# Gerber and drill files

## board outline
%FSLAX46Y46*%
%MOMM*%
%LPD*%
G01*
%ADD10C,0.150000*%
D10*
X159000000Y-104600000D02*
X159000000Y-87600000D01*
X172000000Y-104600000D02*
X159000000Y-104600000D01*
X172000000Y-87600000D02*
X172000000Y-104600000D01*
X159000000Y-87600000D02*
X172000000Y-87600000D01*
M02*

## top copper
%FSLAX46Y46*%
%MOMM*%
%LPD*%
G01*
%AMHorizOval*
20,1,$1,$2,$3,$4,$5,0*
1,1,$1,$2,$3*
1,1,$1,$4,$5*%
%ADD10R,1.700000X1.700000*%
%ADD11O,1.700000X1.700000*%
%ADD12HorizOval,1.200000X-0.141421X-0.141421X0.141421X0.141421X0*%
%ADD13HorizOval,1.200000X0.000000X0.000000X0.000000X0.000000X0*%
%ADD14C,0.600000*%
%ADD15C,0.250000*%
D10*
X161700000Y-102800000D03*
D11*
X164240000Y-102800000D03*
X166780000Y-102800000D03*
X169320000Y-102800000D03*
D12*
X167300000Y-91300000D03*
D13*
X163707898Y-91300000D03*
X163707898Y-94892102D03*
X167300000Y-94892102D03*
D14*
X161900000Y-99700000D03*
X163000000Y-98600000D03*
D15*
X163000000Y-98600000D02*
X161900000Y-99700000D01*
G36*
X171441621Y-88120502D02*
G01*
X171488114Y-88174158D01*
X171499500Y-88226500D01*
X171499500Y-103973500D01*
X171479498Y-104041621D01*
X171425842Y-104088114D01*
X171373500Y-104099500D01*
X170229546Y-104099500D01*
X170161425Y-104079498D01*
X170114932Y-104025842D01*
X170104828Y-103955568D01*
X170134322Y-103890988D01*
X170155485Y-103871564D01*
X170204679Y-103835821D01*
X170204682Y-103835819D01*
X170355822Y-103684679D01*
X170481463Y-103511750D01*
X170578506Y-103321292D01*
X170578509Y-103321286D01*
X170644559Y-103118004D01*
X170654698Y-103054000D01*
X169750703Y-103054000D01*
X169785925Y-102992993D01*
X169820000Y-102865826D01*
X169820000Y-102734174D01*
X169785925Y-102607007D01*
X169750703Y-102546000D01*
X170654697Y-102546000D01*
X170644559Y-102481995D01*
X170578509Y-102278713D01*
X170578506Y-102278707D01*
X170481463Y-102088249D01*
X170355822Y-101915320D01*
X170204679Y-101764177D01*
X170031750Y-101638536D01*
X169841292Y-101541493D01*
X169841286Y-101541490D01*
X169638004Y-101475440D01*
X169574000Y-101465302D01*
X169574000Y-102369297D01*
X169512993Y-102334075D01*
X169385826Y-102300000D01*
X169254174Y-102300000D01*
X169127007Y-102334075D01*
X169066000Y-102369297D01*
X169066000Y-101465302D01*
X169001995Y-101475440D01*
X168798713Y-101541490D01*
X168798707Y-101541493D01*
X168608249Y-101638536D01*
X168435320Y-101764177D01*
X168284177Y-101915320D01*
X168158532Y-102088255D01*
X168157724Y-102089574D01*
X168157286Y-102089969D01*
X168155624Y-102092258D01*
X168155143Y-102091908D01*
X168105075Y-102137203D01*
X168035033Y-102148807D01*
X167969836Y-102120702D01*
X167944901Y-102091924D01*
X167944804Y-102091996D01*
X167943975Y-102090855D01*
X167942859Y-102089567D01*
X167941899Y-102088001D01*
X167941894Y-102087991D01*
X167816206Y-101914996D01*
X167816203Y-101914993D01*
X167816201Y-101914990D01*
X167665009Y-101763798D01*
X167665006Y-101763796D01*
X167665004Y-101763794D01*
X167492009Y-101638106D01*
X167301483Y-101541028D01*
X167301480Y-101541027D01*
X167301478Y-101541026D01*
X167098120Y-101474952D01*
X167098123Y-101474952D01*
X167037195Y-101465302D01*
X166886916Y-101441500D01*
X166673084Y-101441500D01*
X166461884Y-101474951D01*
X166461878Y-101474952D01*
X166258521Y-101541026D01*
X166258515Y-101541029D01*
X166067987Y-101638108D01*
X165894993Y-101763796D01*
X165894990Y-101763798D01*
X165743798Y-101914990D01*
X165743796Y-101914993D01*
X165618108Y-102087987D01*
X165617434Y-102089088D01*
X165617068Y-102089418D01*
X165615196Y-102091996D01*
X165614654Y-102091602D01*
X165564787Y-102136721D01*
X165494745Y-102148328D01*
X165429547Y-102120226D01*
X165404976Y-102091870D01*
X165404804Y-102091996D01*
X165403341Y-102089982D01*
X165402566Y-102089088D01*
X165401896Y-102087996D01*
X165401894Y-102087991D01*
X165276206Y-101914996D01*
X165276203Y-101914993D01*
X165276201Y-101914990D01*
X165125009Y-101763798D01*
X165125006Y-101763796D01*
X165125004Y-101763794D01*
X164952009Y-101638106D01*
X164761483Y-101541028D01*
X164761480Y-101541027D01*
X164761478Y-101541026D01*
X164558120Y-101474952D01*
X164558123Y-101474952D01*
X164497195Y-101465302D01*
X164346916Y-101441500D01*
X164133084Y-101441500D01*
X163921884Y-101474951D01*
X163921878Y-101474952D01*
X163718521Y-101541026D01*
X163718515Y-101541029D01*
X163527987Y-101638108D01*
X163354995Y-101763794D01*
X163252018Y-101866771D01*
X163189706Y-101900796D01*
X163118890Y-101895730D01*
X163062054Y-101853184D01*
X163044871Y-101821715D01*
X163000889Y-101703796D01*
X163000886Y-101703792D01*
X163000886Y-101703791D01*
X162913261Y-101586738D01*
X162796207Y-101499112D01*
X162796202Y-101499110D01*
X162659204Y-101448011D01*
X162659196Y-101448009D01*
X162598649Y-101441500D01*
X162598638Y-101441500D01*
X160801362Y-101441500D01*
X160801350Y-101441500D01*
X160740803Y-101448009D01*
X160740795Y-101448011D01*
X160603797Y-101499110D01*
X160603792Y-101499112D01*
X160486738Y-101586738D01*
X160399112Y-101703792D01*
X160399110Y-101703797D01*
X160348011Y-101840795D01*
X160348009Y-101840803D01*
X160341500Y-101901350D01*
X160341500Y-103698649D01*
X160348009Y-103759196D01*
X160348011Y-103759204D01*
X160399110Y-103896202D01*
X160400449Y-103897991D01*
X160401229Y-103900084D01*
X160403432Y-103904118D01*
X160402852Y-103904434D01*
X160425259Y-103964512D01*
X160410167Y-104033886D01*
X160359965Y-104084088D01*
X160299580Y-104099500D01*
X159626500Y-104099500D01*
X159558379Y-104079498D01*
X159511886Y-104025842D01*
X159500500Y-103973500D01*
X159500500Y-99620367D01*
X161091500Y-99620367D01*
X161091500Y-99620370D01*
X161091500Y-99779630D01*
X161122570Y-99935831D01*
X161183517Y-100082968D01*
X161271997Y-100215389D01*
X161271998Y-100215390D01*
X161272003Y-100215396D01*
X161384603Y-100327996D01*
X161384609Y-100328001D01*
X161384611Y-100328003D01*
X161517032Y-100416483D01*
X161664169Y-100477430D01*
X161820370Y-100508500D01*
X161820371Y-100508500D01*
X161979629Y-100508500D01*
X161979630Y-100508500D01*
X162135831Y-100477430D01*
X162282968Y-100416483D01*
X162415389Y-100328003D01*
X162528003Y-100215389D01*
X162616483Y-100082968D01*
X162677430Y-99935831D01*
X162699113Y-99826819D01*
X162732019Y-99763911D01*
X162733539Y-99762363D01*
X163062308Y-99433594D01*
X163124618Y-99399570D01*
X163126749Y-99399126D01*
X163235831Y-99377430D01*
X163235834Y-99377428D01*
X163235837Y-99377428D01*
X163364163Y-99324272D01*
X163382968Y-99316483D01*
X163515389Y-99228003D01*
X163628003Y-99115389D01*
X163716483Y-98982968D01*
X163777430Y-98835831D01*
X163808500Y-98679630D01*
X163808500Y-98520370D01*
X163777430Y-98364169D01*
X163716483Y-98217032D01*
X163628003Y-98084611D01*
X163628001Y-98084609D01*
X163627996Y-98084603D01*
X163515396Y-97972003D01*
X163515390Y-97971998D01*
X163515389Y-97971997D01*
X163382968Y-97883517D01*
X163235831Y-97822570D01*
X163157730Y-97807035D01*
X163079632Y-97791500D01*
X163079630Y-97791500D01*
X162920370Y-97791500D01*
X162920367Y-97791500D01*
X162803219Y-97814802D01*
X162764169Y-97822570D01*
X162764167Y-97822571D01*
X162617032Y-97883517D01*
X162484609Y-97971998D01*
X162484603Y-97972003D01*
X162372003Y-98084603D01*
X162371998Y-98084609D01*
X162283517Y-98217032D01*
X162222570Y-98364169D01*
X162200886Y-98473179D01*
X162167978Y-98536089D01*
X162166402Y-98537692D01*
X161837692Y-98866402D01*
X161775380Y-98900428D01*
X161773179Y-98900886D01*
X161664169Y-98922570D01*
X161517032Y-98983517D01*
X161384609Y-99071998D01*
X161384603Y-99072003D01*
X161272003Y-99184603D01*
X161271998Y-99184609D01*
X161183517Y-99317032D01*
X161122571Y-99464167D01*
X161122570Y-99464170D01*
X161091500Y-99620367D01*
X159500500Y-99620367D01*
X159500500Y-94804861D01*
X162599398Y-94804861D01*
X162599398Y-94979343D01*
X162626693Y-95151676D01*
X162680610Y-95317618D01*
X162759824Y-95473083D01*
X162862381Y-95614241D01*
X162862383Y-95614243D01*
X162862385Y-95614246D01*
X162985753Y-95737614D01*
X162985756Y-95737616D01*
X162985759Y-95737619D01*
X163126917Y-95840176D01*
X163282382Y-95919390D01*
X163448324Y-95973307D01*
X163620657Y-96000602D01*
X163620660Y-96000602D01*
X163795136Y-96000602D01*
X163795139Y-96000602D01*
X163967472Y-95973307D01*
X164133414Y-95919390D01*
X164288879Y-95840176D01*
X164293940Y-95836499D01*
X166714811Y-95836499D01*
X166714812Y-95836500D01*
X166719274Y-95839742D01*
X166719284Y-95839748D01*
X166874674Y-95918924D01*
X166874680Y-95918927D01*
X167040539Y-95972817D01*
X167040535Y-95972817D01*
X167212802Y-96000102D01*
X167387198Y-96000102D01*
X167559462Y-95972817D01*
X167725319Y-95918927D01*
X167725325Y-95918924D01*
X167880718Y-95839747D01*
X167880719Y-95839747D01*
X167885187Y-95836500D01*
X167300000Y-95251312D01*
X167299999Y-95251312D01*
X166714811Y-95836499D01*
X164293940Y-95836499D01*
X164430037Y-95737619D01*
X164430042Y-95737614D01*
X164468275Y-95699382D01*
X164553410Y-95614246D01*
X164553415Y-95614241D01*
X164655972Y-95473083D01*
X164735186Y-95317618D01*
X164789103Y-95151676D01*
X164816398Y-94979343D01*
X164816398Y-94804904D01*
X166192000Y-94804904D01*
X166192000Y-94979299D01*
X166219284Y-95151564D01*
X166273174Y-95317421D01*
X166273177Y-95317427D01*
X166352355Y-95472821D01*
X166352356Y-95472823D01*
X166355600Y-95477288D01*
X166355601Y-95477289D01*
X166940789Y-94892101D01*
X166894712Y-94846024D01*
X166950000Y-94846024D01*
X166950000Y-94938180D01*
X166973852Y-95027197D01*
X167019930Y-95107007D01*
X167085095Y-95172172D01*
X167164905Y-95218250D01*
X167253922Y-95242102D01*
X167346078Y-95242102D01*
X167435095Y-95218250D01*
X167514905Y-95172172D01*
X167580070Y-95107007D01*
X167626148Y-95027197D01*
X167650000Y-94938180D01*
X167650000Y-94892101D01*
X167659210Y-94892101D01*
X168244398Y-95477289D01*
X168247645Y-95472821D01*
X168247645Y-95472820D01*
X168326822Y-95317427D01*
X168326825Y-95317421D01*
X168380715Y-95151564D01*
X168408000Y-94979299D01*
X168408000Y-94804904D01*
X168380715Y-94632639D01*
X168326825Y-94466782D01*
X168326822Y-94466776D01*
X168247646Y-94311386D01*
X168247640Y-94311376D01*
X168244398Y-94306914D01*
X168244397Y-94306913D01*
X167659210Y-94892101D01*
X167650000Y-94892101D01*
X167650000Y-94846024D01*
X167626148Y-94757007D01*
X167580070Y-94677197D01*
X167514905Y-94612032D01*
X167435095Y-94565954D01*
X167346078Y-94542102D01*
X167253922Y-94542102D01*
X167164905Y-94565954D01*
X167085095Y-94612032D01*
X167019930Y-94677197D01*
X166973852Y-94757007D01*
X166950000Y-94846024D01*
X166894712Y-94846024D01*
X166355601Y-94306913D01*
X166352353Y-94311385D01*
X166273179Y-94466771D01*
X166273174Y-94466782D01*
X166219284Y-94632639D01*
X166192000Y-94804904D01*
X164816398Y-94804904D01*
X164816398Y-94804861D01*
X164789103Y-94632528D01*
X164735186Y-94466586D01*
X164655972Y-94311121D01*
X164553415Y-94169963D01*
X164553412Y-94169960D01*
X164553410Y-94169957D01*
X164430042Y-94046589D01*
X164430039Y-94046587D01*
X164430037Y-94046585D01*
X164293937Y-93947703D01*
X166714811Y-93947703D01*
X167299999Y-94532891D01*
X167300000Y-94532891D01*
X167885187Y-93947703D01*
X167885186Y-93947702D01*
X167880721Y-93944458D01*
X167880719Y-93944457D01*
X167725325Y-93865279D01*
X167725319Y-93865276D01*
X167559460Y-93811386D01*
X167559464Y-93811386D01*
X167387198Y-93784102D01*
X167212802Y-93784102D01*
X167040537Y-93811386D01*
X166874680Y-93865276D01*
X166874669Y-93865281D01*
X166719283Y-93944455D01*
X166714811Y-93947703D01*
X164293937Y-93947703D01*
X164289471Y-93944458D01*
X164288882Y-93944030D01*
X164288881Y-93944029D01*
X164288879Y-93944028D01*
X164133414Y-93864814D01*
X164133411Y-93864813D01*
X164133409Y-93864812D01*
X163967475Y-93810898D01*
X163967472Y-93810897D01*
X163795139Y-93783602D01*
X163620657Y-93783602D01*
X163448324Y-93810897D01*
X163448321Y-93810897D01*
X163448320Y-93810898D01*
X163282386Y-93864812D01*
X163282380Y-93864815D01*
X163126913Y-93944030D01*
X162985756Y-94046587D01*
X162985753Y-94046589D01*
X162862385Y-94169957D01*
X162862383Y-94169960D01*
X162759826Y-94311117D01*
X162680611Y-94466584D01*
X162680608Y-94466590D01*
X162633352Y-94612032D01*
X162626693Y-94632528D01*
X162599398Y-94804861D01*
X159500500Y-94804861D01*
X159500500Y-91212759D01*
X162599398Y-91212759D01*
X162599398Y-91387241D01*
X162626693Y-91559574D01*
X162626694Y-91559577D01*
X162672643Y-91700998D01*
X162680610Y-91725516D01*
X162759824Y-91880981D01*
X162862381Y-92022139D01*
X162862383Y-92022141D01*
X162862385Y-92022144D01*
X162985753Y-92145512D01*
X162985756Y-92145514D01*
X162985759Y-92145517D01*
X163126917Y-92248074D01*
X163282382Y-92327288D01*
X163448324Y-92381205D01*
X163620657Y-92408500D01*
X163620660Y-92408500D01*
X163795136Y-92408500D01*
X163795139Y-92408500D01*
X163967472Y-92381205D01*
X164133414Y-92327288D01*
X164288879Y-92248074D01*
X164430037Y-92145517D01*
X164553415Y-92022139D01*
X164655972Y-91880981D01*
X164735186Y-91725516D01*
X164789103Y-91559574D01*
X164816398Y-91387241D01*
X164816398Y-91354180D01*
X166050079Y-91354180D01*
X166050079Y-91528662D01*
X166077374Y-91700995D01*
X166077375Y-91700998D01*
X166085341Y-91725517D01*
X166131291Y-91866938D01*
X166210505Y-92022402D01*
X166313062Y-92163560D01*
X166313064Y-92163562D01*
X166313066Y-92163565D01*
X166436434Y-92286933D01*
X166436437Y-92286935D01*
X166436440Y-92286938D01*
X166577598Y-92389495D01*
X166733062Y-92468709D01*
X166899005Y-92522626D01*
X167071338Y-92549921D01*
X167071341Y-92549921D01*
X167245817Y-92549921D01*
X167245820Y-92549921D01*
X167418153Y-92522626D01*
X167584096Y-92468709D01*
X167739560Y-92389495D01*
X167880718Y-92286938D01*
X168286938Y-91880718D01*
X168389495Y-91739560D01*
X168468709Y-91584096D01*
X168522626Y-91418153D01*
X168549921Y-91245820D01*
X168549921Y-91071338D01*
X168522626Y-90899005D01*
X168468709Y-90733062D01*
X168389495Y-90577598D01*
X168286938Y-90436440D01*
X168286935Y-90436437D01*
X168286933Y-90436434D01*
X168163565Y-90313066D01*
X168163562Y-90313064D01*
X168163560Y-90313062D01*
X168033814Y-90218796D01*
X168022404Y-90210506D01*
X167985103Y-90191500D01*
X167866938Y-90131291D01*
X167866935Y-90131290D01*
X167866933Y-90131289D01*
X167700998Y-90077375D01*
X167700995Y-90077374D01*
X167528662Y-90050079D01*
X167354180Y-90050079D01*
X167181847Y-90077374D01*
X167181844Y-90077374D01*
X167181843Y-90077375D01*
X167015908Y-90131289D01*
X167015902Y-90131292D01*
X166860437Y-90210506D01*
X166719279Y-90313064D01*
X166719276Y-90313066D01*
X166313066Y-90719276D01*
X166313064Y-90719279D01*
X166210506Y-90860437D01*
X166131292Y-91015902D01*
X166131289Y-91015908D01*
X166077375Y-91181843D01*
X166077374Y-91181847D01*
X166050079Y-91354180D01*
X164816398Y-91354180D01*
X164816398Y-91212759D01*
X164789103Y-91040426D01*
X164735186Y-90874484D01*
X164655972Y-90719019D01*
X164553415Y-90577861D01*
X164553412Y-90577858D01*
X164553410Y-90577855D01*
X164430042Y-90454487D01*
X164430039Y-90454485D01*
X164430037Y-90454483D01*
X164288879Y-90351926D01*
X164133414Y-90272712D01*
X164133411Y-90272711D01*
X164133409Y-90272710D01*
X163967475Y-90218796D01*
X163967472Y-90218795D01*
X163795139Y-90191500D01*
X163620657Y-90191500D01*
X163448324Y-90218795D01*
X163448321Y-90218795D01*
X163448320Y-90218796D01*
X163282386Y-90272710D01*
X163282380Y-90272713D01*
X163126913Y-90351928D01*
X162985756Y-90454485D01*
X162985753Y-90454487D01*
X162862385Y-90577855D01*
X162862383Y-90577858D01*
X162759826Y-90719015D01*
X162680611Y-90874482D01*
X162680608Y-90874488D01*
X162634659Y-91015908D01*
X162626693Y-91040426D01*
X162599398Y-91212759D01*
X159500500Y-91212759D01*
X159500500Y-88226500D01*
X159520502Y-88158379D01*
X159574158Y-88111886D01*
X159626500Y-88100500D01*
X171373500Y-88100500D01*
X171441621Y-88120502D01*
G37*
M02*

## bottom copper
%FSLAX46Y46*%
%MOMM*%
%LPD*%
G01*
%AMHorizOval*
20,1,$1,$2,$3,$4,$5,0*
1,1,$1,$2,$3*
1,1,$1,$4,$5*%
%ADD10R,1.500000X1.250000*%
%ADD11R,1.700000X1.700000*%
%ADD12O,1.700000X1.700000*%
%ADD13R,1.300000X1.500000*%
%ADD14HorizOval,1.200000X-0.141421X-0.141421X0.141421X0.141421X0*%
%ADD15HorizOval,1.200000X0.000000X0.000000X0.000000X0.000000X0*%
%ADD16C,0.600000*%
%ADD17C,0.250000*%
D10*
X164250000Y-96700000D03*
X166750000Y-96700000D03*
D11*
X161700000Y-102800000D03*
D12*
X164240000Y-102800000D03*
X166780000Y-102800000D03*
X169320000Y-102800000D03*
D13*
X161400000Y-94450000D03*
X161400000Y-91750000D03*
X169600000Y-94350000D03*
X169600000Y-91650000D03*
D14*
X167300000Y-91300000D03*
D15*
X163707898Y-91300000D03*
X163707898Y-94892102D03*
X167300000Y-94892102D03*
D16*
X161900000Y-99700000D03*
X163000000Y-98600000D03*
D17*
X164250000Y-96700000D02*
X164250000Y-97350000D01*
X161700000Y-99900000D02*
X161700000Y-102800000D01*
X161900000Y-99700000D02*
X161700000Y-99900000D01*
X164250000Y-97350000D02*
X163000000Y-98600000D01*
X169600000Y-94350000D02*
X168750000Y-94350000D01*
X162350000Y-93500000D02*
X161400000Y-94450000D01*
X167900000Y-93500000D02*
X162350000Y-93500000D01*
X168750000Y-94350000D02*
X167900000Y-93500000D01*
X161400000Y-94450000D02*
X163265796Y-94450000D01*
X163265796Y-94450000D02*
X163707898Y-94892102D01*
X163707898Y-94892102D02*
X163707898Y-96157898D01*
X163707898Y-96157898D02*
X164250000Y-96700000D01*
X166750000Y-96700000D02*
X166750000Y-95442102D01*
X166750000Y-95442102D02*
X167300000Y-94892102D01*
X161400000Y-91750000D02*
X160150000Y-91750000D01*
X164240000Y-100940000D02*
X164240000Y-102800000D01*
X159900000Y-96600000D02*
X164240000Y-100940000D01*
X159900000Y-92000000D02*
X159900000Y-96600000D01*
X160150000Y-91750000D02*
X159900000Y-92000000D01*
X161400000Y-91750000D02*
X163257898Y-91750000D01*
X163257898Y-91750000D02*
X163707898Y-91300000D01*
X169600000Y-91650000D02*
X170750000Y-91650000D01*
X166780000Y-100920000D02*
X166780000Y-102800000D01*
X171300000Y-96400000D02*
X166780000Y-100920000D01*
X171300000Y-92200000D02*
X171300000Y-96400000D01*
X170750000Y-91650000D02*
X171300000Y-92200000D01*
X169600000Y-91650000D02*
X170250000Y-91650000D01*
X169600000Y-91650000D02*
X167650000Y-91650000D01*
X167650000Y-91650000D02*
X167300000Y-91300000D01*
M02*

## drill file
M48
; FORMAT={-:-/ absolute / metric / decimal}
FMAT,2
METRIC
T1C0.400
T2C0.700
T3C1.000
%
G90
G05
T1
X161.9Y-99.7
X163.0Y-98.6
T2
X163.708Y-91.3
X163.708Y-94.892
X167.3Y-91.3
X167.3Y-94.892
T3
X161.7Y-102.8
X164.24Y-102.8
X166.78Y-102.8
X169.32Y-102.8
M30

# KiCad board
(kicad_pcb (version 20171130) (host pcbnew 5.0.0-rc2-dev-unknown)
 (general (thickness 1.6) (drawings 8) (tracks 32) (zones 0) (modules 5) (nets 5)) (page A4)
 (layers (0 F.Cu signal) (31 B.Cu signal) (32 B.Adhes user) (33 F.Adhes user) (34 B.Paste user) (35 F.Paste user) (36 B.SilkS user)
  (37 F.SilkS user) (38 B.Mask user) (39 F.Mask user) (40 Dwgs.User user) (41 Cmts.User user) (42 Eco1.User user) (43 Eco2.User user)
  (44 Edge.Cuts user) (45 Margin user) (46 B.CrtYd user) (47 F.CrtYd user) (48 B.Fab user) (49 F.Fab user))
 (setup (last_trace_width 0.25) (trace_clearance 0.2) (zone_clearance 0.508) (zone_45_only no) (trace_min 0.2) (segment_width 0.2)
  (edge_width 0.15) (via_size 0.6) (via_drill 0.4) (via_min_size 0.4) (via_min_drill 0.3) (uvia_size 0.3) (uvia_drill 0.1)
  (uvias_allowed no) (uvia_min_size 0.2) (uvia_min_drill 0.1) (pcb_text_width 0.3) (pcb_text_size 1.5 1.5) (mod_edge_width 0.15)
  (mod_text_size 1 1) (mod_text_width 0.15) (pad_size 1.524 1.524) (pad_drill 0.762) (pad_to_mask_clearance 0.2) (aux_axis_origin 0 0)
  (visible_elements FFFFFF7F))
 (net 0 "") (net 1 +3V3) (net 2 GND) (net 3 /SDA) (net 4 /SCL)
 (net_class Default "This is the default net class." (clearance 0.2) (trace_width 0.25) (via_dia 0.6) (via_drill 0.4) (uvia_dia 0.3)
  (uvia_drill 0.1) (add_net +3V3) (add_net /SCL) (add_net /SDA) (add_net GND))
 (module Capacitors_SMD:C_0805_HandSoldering (layer B.Cu) (at 165.5 96.7)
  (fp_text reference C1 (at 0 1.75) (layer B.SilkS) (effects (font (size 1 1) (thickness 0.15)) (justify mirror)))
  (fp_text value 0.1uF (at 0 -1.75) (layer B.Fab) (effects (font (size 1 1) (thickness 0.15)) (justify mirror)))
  (pad 1 smd rect (at -1.25 0) (size 1.5 1.25) (layers B.Cu B.Paste B.Mask) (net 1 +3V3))
  (pad 2 smd rect (at 1.25 0) (size 1.5 1.25) (layers B.Cu B.Paste B.Mask) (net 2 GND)))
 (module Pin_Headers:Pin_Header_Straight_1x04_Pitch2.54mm (layer F.Cu) (at 161.7 102.8 90)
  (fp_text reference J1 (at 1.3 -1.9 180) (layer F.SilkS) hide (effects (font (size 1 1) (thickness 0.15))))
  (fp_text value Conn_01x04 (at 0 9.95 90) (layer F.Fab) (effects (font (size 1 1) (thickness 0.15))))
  (pad 1 thru_hole rect (at 0 0 90) (size 1.7 1.7) (drill 1) (layers *.Cu *.Mask) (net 1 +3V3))
  (pad 2 thru_hole oval (at 0 2.54 90) (size 1.7 1.7) (drill 1) (layers *.Cu *.Mask) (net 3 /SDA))
  (pad 3 thru_hole oval (at 0 5.08 90) (size 1.7 1.7) (drill 1) (layers *.Cu *.Mask) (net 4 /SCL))
  (pad 4 thru_hole oval (at 0 7.62 90) (size 1.7 1.7) (drill 1) (layers *.Cu *.Mask) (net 2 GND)))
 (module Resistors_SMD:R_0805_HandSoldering (layer B.Cu) (at 161.4 93.1 90)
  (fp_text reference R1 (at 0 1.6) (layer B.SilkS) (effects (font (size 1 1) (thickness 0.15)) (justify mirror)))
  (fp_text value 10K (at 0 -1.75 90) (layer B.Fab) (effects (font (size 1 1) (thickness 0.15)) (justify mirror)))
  (pad 1 smd rect (at -1.35 0 90) (size 1.5 1.3) (layers B.Cu B.Paste B.Mask) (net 1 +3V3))
  (pad 2 smd rect (at 1.35 0 90) (size 1.5 1.3) (layers B.Cu B.Paste B.Mask) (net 3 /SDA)))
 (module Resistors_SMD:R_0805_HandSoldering (layer B.Cu) (at 169.6 93 90)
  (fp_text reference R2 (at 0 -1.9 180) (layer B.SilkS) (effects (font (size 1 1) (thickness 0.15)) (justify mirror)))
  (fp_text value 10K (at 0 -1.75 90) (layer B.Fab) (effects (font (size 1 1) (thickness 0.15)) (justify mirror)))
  (pad 1 smd rect (at -1.35 0 90) (size 1.5 1.3) (layers B.Cu B.Paste B.Mask) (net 1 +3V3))
  (pad 2 smd rect (at 1.35 0 90) (size 1.5 1.3) (layers B.Cu B.Paste B.Mask) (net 4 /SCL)))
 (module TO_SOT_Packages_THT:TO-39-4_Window (layer F.Cu) (at 167.3 91.3 225)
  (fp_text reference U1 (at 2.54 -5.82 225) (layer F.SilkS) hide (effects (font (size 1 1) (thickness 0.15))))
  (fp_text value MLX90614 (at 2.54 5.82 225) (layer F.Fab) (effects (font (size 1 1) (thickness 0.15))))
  (pad 1 thru_hole oval (at 0 0 225) (size 1.6 1.2) (drill 0.7) (layers *.Cu *.Mask) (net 4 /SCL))
  (pad 2 thru_hole oval (at 2.54 2.54 225) (size 1.2 1.2) (drill 0.7) (layers *.Cu *.Mask) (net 3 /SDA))
  (pad 3 thru_hole oval (at 5.079999 0 225) (size 1.2 1.2) (drill 0.7) (layers *.Cu *.Mask) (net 1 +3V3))
  (pad 4 thru_hole oval (at 2.54 -2.54 225) (size 1.2 1.2) (drill 0.7) (layers *.Cu *.Mask) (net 2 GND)))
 (gr_line (start 159 104.6) (end 159 87.6) (angle 90) (layer Edge.Cuts) (width 0.15))
 (gr_line (start 172 104.6) (end 159 104.6) (angle 90) (layer Edge.Cuts) (width 0.15))
 (gr_line (start 172 87.6) (end 172 104.6) (angle 90) (layer Edge.Cuts) (width 0.15))
 (gr_line (start 159 87.6) (end 172 87.6) (angle 90) (layer Edge.Cuts) (width 0.15))
 (segment (start 164.25 96.7) (end 164.25 97.35) (width 0.25) (layer B.Cu) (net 1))
 (segment (start 161.7 99.9) (end 161.7 102.8) (width 0.25) (layer B.Cu) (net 1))
 (segment (start 161.9 99.7) (end 161.7 99.9) (width 0.25) (layer B.Cu) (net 1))
 (via (at 161.9 99.7) (size 0.6) (drill 0.4) (layers F.Cu B.Cu) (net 1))
 (segment (start 163 98.6) (end 161.9 99.7) (width 0.25) (layer F.Cu) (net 1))
 (via (at 163 98.6) (size 0.6) (drill 0.4) (layers F.Cu B.Cu) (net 1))
 (segment (start 164.25 97.35) (end 163 98.6) (width 0.25) (layer B.Cu) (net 1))
 (segment (start 169.6 94.35) (end 168.75 94.35) (width 0.25) (layer B.Cu) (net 1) (status 10))
 (segment (start 162.35 93.5) (end 161.4 94.45) (width 0.25) (layer B.Cu) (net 1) (status 20))
 (segment (start 167.9 93.5) (end 162.35 93.5) (width 0.25) (layer B.Cu) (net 1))
 (segment (start 168.75 94.35) (end 167.9 93.5) (width 0.25) (layer B.Cu) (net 1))
 (segment (start 161.4 94.45) (end 163.265796 94.45) (width 0.25) (layer B.Cu) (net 1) (status 10))
 (segment (start 163.265796 94.45) (end 163.707898 94.892102) (width 0.25) (layer B.Cu) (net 1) (status 20))
 (segment (start 163.707898 94.892102) (end 163.707898 96.157898) (width 0.25) (layer B.Cu) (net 1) (status 30))
 (segment (start 163.707898 96.157898) (end 164.25 96.7) (width 0.25) (layer B.Cu) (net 1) (status 30))
 (segment (start 166.75 96.7) (end 166.75 95.442102) (width 0.25) (layer B.Cu) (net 2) (status 10))
 (segment (start 166.75 95.442102) (end 167.3 94.892102) (width 0.25) (layer B.Cu) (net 2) (status 20))
 (segment (start 161.4 91.75) (end 160.15 91.75) (width 0.25) (layer B.Cu) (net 3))
 (segment (start 164.24 100.94) (end 164.24 102.8) (width 0.25) (layer B.Cu) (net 3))
 (segment (start 159.9 96.6) (end 164.24 100.94) (width 0.25) (layer B.Cu) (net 3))
 (segment (start 159.9 92) (end 159.9 96.6) (width 0.25) (layer B.Cu) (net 3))
 (segment (start 160.15 91.75) (end 159.9 92) (width 0.25) (layer B.Cu) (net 3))
 (segment (start 161.4 91.75) (end 163.257898 91.75) (width 0.25) (layer B.Cu) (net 3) (status 10))
 (segment (start 163.257898 91.75) (end 163.707898 91.3) (width 0.25) (layer B.Cu) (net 3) (status 20))
 (segment (start 169.6 91.65) (end 170.75 91.65) (width 0.25) (layer B.Cu) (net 4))
 (segment (start 166.78 100.92) (end 166.78 102.8) (width 0.25) (layer B.Cu) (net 4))
 (segment (start 171.3 96.4) (end 166.78 100.92) (width 0.25) (layer B.Cu) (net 4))
 (segment (start 171.3 92.2) (end 171.3 96.4) (width 0.25) (layer B.Cu) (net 4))
 (segment (start 170.75 91.65) (end 171.3 92.2) (width 0.25) (layer B.Cu) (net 4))
 (segment (start 169.6 91.65) (end 170.25 91.65) (width 0.25) (layer B.Cu) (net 4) (status 30))
 (segment (start 169.6 91.65) (end 167.65 91.65) (width 0.25) (layer B.Cu) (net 4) (status 30))
 (segment (start 167.65 91.65) (end 167.3 91.3) (width 0.25) (layer B.Cu) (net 4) (status 30))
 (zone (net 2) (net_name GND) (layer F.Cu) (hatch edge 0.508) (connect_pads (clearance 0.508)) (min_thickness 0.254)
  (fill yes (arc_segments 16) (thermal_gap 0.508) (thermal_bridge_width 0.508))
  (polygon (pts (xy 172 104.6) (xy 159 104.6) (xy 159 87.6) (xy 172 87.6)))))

